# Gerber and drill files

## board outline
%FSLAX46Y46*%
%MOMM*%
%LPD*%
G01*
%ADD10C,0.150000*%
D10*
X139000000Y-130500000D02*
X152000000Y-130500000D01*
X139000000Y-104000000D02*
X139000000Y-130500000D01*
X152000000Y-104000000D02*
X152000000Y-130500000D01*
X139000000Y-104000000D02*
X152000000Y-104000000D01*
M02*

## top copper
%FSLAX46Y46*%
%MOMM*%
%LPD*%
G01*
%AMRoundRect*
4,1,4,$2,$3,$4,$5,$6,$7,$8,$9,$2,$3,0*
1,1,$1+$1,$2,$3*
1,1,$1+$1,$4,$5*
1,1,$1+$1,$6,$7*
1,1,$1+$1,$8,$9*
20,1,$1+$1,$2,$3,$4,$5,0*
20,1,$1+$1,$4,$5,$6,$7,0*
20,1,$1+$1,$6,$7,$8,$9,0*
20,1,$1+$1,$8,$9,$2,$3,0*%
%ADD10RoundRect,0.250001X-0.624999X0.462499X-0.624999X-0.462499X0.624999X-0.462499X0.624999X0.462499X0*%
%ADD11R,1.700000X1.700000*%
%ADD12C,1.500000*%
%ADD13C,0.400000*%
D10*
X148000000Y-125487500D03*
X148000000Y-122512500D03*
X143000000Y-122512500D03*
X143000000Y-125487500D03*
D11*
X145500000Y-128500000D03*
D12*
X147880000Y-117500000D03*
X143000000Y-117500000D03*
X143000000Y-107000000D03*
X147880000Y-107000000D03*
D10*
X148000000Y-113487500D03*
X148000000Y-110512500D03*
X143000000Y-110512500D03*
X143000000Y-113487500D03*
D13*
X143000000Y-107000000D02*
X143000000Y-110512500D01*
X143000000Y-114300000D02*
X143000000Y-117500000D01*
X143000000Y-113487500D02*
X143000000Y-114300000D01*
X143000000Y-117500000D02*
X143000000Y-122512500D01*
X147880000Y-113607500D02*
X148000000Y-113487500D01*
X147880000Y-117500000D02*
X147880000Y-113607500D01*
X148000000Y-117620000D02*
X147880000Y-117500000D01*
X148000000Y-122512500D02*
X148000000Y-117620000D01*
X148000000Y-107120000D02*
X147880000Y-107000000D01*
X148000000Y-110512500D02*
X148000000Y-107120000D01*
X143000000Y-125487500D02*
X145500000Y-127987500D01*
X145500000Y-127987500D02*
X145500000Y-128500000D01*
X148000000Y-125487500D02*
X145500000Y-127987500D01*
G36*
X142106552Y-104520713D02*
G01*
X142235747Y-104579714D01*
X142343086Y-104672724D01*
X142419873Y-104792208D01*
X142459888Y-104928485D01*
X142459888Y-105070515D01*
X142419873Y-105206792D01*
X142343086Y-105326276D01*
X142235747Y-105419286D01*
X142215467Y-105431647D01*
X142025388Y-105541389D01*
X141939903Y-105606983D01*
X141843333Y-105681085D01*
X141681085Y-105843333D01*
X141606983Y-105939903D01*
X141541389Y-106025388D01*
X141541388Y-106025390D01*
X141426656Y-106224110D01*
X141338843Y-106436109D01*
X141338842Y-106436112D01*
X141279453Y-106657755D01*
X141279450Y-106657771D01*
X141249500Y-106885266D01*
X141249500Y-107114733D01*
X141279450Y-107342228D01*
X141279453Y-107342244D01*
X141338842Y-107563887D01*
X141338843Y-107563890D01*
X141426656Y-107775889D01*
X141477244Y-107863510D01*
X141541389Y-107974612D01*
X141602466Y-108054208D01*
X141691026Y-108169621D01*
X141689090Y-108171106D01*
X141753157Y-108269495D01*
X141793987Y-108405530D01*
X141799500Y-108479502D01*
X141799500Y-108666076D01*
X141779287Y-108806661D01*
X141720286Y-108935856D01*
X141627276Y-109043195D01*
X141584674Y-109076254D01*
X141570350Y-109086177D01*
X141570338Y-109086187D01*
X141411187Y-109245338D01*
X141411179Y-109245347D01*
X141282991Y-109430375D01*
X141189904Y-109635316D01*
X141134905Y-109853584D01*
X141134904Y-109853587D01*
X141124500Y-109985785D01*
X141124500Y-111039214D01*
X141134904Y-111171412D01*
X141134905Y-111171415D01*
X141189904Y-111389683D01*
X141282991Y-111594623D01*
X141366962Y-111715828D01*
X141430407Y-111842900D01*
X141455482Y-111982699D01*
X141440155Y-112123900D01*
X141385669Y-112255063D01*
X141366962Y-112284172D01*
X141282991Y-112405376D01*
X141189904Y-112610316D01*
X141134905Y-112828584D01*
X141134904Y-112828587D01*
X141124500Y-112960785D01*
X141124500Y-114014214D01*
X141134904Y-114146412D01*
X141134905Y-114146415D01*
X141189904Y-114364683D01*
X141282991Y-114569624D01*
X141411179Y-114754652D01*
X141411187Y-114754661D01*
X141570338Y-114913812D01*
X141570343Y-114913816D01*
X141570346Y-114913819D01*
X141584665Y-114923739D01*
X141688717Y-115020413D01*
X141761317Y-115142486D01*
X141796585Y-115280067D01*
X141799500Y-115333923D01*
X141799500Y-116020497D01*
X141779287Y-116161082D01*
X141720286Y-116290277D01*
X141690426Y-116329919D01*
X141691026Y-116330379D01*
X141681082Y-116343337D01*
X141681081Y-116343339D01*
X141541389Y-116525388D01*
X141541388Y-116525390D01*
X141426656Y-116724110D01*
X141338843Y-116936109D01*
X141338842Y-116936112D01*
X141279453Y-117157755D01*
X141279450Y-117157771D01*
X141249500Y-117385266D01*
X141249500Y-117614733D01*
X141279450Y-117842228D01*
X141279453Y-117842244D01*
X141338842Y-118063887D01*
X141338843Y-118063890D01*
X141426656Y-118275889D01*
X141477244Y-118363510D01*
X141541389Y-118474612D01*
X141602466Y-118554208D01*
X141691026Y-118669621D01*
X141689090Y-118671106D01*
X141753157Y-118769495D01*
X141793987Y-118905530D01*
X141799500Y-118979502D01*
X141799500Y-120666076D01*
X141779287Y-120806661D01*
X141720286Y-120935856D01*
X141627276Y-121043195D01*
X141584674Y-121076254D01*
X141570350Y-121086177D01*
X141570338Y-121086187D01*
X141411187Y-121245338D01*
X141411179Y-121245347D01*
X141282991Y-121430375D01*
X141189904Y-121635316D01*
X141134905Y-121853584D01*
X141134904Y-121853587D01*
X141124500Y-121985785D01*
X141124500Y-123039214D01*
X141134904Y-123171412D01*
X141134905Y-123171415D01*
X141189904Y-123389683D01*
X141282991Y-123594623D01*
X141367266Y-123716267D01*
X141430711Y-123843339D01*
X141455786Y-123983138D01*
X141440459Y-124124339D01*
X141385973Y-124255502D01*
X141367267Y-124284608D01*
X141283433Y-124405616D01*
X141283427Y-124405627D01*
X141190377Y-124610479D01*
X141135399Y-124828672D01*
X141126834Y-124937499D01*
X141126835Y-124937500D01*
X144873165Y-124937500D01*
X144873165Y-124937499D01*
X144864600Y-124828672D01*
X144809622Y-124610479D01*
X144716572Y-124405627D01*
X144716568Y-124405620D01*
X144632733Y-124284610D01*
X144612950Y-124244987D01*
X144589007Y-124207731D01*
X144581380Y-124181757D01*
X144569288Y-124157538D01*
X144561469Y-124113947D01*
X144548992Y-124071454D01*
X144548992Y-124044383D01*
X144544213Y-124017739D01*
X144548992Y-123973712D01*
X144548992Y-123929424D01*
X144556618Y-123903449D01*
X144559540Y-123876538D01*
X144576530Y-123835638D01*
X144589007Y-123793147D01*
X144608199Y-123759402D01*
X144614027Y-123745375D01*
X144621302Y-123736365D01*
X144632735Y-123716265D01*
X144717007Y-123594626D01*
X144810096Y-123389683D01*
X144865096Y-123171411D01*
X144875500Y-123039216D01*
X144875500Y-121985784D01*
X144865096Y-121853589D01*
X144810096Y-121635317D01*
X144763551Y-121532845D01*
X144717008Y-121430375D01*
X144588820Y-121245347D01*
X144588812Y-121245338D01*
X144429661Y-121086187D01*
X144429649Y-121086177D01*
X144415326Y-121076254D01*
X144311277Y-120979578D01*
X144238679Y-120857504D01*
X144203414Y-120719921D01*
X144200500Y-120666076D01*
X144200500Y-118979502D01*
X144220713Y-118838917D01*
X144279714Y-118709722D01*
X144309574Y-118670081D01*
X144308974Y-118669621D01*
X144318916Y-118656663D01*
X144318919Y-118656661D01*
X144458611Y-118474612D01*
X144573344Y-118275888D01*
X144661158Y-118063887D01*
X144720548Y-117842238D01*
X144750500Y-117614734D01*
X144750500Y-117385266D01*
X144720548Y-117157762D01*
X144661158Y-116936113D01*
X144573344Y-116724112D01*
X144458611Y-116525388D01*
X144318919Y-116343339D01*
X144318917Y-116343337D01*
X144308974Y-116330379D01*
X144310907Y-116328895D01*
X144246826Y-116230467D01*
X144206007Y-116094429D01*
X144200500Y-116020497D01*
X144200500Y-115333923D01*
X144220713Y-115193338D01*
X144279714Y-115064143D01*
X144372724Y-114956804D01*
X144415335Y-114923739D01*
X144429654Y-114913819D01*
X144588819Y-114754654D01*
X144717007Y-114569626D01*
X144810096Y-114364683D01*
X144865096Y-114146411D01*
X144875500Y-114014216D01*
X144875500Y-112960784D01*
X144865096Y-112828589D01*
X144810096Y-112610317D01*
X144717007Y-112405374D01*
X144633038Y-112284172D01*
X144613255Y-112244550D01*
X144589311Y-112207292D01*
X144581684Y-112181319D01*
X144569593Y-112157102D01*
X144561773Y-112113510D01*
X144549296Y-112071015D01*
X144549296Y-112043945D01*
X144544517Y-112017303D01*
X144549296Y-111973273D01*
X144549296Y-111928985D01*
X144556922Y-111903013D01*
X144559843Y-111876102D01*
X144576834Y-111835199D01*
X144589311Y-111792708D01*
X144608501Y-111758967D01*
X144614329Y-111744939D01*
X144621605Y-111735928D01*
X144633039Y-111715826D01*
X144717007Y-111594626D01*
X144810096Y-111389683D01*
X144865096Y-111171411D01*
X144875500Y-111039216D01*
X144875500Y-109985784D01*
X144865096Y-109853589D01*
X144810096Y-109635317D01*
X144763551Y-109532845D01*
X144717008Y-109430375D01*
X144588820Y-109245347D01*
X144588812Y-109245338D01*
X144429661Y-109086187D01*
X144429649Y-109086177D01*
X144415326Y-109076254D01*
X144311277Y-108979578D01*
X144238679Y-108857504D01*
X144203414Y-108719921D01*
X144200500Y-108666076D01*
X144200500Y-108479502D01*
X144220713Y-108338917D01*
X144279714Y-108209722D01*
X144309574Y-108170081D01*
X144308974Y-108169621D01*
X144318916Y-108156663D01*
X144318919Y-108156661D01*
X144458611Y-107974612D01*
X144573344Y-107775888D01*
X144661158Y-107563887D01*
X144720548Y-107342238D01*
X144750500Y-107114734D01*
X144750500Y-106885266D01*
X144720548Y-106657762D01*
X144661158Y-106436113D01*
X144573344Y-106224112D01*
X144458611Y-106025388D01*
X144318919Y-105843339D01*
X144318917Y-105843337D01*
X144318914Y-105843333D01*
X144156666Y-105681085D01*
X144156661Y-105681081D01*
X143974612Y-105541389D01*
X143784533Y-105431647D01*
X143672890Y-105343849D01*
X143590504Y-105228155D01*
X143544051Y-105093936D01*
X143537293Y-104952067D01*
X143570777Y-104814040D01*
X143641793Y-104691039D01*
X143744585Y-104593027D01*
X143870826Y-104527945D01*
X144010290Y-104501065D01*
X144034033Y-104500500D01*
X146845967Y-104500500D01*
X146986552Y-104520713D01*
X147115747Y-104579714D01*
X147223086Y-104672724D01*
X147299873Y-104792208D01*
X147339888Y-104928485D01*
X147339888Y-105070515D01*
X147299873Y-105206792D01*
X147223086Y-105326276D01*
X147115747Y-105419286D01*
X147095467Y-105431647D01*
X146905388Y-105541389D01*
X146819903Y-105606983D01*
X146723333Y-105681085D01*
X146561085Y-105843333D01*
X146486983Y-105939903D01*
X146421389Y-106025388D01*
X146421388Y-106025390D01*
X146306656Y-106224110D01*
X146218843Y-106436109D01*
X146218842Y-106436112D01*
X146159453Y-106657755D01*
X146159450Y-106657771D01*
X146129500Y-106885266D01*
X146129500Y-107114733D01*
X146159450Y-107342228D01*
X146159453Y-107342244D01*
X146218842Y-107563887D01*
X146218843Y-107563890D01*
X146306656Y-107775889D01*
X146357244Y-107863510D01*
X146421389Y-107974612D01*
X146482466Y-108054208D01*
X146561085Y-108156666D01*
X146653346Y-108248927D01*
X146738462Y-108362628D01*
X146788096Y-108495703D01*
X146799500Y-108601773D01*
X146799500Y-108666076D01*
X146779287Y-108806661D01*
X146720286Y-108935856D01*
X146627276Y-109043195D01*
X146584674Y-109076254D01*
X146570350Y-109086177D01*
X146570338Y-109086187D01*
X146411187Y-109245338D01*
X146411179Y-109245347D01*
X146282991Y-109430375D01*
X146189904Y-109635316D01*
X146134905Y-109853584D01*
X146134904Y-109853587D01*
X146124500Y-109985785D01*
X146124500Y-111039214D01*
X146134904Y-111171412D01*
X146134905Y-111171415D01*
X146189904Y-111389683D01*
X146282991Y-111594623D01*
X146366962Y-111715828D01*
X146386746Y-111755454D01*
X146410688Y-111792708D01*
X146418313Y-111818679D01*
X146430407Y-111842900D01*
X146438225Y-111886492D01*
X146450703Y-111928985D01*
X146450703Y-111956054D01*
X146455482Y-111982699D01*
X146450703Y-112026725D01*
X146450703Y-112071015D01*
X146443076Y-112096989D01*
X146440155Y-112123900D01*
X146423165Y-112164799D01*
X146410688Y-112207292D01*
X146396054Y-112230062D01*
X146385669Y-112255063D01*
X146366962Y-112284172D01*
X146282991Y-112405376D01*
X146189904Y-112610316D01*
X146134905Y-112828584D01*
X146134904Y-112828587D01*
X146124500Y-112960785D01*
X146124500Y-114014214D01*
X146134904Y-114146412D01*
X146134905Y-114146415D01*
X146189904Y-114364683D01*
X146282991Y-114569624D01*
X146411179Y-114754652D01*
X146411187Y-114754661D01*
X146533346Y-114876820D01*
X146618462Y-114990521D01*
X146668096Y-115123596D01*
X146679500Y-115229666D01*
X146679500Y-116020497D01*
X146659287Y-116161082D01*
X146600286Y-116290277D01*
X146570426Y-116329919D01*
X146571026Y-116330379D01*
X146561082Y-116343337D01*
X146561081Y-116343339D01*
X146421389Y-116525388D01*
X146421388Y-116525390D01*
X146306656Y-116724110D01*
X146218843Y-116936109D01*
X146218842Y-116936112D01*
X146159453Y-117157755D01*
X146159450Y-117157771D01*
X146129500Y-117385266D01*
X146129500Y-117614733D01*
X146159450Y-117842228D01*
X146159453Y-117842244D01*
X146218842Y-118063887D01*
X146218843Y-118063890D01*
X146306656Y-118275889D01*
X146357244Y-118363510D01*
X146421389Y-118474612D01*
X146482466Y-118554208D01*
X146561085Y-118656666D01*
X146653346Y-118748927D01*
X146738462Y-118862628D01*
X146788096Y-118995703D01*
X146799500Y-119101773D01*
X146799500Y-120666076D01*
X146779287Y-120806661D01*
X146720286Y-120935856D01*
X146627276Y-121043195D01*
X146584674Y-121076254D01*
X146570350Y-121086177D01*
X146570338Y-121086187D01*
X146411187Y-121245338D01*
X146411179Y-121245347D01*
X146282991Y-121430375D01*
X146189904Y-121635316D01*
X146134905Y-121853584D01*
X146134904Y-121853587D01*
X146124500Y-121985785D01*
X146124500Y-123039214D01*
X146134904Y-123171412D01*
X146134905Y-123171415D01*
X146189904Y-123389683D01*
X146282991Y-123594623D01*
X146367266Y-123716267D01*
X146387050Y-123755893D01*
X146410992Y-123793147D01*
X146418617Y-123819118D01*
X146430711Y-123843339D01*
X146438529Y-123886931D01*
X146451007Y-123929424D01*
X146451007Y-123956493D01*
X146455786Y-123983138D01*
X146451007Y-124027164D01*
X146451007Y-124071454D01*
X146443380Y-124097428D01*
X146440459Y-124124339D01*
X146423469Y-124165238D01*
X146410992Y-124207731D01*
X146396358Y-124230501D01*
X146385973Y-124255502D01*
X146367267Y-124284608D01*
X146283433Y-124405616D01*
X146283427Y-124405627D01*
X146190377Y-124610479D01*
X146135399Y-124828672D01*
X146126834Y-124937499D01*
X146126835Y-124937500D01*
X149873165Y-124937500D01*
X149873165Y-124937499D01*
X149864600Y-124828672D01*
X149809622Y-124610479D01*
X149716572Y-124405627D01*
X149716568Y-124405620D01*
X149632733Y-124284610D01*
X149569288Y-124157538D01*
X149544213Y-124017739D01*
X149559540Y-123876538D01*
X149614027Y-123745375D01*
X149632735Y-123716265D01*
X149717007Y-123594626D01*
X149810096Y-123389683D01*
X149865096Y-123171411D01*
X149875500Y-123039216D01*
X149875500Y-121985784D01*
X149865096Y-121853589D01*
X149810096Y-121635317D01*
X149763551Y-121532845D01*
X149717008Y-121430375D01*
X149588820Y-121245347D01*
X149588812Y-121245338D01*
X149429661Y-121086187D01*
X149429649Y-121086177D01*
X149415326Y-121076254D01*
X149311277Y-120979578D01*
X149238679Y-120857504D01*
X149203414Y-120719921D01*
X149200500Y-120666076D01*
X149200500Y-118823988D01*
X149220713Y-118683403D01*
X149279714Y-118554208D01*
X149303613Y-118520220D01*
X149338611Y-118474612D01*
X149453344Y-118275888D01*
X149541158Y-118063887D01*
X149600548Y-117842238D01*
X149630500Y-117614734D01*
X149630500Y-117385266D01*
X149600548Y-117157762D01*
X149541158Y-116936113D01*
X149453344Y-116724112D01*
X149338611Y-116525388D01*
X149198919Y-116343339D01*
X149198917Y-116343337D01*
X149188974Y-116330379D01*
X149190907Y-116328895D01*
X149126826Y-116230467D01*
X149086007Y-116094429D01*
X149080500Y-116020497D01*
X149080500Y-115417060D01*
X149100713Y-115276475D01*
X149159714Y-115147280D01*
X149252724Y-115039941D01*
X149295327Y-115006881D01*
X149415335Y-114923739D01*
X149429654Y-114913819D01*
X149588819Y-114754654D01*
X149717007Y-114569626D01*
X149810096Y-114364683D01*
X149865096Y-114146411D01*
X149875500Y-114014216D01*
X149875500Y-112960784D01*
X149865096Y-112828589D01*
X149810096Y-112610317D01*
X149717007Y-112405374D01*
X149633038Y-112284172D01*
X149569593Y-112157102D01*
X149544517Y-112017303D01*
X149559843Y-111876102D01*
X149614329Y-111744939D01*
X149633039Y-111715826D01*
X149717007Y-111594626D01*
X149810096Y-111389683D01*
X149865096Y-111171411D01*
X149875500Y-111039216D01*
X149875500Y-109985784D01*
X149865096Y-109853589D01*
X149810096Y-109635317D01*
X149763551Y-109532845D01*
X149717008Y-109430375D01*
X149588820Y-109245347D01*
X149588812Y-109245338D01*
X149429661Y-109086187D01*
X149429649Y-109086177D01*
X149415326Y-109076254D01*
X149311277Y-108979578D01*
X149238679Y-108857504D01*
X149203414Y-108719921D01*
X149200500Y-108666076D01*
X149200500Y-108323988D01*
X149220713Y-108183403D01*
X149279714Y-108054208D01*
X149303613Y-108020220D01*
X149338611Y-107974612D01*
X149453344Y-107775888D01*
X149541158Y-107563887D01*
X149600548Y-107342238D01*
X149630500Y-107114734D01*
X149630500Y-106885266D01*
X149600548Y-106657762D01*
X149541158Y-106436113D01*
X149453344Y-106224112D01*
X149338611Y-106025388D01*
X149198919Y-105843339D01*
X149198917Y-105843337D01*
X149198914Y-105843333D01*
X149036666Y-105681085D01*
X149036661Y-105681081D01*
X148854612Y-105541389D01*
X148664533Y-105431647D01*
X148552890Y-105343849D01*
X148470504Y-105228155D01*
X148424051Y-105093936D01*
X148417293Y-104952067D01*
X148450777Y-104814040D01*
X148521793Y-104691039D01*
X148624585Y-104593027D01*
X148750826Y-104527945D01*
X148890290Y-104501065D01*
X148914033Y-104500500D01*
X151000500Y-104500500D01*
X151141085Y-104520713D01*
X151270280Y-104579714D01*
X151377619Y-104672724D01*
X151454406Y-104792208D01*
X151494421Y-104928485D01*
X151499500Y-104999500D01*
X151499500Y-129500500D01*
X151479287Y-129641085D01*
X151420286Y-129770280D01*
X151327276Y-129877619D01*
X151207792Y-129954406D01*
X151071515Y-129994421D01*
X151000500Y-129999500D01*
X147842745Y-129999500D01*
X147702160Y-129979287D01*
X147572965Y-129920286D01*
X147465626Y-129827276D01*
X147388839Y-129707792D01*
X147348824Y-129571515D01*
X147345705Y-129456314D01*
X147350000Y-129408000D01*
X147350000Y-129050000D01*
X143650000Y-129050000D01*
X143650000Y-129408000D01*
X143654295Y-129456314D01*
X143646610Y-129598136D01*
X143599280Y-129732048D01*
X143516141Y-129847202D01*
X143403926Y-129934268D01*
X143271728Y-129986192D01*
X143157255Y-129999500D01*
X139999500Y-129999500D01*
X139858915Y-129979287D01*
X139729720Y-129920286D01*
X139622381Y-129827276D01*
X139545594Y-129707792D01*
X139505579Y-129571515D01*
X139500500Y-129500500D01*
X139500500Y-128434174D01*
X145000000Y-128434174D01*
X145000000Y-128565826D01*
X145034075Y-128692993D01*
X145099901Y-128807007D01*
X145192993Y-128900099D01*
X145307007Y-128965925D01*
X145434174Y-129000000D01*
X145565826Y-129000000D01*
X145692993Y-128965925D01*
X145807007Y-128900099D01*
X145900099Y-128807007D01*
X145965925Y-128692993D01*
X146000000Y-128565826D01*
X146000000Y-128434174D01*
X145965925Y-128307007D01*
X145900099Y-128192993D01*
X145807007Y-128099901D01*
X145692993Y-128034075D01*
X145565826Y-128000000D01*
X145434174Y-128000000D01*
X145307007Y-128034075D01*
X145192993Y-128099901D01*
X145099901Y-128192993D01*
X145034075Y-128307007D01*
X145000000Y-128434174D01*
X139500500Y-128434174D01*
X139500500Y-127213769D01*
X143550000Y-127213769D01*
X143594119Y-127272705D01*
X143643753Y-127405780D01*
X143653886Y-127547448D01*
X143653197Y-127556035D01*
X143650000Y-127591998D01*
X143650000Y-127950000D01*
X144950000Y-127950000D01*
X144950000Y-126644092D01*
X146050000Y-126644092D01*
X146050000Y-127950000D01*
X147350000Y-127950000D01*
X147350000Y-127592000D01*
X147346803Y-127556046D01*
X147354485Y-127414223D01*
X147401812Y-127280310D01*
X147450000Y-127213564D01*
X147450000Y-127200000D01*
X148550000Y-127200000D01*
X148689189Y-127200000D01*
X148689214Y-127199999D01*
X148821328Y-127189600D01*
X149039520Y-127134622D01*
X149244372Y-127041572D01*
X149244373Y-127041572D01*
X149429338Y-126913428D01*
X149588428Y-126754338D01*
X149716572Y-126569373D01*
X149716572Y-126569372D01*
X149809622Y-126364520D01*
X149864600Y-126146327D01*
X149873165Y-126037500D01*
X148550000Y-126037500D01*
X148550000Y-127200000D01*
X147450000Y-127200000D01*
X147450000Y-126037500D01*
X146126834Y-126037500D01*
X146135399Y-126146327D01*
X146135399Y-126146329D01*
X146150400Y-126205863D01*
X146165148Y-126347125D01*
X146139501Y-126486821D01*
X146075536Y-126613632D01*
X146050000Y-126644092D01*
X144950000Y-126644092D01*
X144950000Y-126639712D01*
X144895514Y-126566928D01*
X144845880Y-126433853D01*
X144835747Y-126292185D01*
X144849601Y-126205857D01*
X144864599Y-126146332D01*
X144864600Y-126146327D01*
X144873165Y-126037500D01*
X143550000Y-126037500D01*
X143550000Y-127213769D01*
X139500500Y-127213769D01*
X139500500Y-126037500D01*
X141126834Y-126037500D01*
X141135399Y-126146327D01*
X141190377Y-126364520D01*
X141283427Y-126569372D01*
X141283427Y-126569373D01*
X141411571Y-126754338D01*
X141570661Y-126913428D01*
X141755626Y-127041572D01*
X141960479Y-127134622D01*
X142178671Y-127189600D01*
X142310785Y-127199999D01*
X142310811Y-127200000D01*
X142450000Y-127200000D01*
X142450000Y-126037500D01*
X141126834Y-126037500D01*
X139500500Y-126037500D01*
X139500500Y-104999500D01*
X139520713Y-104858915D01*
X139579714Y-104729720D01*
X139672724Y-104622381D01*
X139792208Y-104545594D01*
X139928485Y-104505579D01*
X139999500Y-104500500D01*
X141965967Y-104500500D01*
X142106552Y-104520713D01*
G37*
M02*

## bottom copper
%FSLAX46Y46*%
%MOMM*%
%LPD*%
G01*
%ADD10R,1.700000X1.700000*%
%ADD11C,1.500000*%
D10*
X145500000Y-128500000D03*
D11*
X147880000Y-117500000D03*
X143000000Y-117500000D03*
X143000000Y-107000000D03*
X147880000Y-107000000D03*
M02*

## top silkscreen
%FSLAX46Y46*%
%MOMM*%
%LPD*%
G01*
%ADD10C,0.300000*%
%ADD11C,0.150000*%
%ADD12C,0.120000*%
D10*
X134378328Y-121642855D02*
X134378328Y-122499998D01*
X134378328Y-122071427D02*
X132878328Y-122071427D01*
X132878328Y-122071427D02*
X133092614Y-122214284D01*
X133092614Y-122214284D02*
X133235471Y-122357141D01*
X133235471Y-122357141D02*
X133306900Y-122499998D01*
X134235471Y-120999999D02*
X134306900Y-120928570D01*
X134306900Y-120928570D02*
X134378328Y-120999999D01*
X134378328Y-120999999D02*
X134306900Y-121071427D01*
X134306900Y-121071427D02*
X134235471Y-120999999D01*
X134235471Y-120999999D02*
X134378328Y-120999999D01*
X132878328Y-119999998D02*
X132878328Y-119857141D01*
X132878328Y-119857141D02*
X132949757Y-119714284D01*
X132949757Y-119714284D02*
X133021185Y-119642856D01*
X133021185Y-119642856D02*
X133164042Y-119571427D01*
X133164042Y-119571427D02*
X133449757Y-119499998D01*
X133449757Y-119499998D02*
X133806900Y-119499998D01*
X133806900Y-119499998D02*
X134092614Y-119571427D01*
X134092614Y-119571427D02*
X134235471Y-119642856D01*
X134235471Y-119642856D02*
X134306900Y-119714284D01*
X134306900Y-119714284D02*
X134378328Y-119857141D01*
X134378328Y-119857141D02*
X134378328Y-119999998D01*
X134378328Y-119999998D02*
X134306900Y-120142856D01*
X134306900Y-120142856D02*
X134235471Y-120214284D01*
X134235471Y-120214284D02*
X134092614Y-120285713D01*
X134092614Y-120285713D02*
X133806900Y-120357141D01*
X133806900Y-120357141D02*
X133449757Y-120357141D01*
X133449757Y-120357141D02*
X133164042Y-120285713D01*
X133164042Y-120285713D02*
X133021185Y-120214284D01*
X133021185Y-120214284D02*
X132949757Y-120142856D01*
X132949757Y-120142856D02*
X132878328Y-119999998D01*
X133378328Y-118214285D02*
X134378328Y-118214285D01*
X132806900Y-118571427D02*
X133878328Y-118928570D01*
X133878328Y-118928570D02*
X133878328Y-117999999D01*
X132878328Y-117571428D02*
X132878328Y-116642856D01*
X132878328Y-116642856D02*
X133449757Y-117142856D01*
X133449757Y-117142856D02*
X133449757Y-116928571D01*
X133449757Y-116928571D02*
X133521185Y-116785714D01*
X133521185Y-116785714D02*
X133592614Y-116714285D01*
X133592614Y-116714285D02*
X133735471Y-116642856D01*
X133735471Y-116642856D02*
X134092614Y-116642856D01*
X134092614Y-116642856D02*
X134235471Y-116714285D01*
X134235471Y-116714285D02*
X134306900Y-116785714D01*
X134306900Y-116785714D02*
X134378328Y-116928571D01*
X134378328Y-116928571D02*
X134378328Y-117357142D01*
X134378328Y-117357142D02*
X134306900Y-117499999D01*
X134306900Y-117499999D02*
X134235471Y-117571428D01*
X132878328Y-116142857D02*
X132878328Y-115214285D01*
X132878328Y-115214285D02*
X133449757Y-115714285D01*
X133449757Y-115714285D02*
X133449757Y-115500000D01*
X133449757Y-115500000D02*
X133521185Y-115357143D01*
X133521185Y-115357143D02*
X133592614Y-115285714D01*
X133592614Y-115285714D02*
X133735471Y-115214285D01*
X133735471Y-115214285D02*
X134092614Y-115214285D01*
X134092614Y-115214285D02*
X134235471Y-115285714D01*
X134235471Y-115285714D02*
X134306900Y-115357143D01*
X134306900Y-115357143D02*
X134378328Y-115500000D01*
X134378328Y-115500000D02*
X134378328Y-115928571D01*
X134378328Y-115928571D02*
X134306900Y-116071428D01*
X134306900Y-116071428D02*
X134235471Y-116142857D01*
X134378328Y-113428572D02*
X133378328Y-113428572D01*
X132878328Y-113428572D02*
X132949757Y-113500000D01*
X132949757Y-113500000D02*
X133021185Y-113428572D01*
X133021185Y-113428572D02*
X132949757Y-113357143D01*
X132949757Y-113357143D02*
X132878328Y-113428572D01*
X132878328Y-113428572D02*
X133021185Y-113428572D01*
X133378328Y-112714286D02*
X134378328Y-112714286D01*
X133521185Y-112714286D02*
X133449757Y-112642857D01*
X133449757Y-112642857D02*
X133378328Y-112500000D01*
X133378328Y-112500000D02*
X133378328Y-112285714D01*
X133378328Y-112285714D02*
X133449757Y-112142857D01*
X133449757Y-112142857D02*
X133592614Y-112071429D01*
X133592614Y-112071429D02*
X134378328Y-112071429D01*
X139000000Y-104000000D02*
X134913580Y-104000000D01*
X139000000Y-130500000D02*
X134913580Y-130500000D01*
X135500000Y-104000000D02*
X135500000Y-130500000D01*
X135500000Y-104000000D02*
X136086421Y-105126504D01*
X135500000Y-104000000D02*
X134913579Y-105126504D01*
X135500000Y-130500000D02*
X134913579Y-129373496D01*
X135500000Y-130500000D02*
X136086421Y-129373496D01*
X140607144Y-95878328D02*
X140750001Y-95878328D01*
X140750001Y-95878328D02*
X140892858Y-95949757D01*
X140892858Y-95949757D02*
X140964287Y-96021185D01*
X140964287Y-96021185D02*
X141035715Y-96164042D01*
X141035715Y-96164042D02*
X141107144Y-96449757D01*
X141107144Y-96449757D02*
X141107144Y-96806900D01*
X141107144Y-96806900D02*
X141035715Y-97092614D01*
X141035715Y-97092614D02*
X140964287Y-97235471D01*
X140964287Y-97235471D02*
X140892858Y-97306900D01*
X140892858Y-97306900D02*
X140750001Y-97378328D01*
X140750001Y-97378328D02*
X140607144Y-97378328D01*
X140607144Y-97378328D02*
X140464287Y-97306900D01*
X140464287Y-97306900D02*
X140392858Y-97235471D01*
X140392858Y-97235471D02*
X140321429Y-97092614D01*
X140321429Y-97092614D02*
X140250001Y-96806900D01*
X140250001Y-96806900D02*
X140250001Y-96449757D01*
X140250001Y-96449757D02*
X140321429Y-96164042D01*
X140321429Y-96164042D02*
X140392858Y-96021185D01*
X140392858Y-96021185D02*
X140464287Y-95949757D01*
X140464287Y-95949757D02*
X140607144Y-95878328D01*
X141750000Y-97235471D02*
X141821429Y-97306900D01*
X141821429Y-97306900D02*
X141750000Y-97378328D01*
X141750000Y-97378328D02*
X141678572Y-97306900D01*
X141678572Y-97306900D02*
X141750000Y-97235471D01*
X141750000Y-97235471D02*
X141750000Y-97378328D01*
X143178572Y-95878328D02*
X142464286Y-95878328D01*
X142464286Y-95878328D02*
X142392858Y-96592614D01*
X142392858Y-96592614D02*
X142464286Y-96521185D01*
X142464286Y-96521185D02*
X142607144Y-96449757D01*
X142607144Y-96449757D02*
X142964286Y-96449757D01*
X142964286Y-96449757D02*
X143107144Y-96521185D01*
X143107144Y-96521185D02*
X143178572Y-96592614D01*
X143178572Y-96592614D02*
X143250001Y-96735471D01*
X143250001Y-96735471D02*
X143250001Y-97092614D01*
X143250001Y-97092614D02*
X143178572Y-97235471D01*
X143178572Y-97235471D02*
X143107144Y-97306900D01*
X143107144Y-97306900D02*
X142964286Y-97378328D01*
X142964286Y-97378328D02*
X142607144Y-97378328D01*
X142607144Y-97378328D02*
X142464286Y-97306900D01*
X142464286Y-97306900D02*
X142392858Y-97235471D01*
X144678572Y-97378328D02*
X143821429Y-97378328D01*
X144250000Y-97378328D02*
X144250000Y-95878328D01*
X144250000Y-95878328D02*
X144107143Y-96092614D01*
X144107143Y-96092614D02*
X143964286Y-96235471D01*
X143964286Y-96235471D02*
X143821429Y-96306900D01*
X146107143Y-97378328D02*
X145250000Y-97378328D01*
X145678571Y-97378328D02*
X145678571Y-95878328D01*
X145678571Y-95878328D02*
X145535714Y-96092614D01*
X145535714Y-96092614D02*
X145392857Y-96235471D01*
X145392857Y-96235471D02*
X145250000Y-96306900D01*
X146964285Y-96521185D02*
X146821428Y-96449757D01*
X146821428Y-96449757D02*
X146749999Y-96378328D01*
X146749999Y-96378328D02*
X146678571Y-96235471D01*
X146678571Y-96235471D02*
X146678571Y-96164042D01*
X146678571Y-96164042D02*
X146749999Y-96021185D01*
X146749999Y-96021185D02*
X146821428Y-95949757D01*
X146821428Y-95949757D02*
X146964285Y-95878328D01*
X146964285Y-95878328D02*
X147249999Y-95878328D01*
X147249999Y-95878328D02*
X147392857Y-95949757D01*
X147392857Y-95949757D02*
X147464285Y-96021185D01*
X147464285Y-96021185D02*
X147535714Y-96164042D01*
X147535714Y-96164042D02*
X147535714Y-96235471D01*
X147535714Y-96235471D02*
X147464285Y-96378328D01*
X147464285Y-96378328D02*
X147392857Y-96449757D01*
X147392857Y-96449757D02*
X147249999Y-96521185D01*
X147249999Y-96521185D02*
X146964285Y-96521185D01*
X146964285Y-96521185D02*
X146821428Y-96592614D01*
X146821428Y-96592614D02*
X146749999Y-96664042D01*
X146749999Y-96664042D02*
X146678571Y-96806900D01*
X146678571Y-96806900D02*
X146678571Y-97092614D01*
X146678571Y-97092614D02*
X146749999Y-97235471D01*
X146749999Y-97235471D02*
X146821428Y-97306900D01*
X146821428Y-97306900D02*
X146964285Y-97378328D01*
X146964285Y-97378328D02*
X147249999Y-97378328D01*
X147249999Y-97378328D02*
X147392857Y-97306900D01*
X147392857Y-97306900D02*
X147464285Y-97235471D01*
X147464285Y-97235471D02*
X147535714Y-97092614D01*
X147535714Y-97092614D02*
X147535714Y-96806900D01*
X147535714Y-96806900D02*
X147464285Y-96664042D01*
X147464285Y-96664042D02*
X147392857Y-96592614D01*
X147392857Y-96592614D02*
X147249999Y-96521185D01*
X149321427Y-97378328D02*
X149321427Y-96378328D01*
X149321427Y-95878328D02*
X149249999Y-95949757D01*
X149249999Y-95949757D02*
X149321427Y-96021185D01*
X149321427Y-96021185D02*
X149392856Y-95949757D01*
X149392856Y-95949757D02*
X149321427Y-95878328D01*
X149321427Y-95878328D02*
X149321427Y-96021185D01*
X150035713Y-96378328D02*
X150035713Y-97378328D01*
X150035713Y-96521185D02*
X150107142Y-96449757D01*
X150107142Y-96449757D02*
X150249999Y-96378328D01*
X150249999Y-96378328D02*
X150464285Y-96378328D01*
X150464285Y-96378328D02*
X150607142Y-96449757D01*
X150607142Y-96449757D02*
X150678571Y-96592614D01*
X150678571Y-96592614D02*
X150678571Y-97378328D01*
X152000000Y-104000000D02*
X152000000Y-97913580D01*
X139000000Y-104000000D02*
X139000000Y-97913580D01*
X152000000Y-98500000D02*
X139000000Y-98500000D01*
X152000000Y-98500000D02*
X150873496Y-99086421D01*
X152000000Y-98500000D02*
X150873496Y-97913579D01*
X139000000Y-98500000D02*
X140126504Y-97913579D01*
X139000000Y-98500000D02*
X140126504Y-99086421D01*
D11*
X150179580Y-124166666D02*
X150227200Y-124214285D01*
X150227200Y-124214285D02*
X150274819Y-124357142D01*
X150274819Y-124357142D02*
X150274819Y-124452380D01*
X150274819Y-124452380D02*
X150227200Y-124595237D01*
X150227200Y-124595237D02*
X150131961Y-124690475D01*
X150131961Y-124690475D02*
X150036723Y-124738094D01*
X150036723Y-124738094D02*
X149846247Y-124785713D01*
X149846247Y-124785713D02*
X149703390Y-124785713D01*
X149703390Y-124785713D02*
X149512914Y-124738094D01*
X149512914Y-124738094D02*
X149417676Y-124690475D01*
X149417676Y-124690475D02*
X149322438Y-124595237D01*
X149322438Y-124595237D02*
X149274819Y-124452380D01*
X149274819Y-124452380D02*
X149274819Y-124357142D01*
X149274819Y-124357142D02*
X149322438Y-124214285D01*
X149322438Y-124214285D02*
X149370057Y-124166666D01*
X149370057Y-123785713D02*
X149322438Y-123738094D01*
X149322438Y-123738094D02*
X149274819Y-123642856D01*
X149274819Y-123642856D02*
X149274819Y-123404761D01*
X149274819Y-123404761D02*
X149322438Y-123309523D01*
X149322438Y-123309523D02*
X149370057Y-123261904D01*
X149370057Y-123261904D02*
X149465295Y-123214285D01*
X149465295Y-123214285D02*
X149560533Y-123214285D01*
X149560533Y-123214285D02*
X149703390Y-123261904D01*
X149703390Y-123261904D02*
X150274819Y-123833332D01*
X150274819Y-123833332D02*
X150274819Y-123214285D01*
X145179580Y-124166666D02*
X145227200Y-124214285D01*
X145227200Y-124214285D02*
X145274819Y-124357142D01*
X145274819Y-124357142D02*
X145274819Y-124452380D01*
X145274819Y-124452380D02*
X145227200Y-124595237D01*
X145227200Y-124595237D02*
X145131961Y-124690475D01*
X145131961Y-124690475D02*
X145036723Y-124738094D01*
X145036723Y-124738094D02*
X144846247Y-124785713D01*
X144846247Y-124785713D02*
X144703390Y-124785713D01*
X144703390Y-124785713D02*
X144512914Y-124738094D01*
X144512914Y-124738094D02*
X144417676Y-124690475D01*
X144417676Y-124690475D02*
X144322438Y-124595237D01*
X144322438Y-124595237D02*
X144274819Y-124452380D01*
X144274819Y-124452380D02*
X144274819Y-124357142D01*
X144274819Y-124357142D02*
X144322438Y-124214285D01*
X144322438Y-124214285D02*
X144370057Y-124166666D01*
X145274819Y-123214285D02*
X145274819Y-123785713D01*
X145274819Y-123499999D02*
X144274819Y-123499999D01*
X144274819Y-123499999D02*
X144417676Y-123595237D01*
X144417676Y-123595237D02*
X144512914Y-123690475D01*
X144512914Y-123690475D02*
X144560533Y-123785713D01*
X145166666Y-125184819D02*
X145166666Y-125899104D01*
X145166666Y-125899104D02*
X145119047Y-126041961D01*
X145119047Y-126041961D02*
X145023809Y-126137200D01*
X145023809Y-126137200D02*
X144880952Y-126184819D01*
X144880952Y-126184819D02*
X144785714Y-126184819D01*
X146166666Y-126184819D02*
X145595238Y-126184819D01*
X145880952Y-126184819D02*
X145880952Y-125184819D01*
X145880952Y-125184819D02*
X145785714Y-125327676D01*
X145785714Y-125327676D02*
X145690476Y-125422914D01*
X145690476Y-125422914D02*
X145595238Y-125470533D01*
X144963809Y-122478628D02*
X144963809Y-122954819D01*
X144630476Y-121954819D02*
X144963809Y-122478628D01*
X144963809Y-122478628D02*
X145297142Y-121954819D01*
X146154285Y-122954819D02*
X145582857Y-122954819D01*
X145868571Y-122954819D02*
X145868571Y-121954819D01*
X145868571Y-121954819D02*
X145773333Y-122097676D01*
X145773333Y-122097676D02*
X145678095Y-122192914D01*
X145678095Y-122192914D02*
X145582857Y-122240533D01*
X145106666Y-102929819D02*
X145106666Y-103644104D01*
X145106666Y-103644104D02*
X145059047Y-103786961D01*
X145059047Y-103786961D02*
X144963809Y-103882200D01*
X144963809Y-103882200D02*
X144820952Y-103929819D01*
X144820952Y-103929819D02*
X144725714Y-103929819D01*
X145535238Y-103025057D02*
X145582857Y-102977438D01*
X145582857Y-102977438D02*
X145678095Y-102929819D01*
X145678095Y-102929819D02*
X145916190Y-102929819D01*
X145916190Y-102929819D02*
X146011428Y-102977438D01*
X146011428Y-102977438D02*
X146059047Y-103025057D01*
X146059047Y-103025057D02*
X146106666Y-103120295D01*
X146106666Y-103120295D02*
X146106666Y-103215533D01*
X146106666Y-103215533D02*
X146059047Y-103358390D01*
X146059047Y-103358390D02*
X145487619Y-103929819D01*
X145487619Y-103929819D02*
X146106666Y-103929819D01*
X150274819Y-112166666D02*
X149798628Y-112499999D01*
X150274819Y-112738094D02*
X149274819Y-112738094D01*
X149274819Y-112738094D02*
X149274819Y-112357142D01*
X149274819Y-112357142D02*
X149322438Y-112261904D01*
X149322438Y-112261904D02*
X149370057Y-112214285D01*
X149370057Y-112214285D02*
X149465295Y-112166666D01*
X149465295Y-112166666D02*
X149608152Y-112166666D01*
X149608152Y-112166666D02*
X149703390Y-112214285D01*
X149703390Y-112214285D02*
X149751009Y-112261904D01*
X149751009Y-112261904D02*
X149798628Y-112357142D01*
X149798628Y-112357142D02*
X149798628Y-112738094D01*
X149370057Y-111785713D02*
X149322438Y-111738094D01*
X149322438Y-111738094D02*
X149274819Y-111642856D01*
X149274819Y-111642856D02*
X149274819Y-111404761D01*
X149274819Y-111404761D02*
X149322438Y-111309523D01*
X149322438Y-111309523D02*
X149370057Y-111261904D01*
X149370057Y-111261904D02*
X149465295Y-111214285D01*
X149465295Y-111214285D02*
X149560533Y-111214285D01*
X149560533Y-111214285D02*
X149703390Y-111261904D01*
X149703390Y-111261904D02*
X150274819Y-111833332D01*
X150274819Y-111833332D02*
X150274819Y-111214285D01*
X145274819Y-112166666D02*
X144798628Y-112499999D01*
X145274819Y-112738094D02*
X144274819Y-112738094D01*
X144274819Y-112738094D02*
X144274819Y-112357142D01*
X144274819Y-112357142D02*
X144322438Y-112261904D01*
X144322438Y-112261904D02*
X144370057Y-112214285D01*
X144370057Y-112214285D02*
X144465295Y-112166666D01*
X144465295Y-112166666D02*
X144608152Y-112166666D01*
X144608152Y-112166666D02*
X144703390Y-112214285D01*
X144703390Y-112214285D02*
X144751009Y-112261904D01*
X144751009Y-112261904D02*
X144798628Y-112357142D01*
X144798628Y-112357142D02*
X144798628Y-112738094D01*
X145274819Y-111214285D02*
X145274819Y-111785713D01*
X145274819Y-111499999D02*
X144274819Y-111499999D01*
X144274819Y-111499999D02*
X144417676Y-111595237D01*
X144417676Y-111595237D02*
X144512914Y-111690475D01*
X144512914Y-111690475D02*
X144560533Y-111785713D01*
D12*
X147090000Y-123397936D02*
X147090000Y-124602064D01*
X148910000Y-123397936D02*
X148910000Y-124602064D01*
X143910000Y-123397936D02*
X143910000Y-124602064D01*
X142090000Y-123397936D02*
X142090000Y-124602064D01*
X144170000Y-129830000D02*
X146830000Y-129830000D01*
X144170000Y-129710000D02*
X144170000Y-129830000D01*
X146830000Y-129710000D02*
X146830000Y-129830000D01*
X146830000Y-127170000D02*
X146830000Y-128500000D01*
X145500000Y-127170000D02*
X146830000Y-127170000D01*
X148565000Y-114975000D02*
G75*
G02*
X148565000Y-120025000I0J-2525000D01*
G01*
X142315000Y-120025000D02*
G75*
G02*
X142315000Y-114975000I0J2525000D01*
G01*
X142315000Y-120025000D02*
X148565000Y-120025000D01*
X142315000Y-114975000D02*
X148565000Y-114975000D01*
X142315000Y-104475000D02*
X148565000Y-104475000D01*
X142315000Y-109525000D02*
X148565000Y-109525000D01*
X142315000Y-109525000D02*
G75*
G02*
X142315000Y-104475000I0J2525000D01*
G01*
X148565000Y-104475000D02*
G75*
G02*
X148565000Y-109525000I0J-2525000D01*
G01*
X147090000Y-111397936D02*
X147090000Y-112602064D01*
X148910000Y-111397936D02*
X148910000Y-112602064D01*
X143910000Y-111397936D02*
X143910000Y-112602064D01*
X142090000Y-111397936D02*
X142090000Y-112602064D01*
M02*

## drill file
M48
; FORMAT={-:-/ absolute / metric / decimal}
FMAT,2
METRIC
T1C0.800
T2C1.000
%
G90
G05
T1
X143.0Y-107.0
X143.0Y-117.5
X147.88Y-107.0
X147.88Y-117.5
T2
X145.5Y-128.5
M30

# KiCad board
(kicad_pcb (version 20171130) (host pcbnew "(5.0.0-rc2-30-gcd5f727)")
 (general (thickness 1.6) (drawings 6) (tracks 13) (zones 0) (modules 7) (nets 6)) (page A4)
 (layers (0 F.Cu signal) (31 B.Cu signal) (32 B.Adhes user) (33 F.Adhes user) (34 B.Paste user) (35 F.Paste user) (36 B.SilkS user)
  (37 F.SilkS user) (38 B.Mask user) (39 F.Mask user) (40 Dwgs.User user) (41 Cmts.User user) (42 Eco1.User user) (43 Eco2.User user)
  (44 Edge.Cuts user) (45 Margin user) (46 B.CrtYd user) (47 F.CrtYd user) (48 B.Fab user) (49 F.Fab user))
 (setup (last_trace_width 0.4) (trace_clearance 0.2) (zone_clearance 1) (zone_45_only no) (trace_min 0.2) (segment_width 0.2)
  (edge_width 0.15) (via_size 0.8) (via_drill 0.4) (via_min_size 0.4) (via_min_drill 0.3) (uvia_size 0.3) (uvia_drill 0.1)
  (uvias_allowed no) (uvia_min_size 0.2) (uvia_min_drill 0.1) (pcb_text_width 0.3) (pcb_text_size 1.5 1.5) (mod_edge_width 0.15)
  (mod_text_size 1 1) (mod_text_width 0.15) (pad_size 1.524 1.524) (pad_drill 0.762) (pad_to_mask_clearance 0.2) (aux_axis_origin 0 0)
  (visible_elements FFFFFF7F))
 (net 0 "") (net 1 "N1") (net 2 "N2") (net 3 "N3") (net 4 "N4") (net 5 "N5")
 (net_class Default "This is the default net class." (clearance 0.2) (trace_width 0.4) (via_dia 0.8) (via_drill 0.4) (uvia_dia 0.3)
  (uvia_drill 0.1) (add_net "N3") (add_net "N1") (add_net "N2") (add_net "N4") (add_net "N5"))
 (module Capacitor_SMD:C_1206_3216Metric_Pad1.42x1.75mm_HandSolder (layer F.Cu) (at 148 124 270)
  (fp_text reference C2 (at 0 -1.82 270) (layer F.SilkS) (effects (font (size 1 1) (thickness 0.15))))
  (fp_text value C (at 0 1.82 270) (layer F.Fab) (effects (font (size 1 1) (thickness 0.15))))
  (fp_line (start -0.602064 0.91) (end 0.602064 0.91) (layer F.SilkS) (width 0.12))
  (fp_line (start -0.602064 -0.91) (end 0.602064 -0.91) (layer F.SilkS) (width 0.12))
  (pad 2 smd roundrect (at 1.4875 0 270) (size 1.425 1.75) (layers F.Cu F.Paste F.Mask) (roundrect_rratio 0.175439) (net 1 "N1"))
  (pad 1 smd roundrect (at -1.4875 0 270) (size 1.425 1.75) (layers F.Cu F.Paste F.Mask) (roundrect_rratio 0.175439) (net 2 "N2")))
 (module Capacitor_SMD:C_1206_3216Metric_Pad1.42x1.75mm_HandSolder (layer F.Cu) (at 143 124 270)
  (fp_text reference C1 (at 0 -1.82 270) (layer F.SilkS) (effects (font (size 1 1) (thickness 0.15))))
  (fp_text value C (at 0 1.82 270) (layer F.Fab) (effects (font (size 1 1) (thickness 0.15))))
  (fp_line (start -0.602064 -0.91) (end 0.602064 -0.91) (layer F.SilkS) (width 0.12))
  (fp_line (start -0.602064 0.91) (end 0.602064 0.91) (layer F.SilkS) (width 0.12))
  (pad 1 smd roundrect (at -1.4875 0 270) (size 1.425 1.75) (layers F.Cu F.Paste F.Mask) (roundrect_rratio 0.175439) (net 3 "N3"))
  (pad 2 smd roundrect (at 1.4875 0 270) (size 1.425 1.75) (layers F.Cu F.Paste F.Mask) (roundrect_rratio 0.175439) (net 1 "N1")))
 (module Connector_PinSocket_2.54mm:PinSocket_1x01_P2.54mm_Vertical (layer F.Cu) (at 145.5 128.5)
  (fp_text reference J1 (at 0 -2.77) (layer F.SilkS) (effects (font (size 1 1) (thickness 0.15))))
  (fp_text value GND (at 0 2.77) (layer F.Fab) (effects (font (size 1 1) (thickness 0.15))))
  (fp_line (start -1.33 1.33) (end 1.33 1.33) (layer F.SilkS) (width 0.12))
  (fp_line (start -1.33 1.21) (end -1.33 1.33) (layer F.SilkS) (width 0.12))
  (fp_line (start 1.33 1.21) (end 1.33 1.33) (layer F.SilkS) (width 0.12))
  (fp_line (start 1.33 -1.33) (end 1.33 0) (layer F.SilkS) (width 0.12))
  (fp_line (start 0 -1.33) (end 1.33 -1.33) (layer F.SilkS) (width 0.12))
  (pad 1 thru_hole rect (at 0 0) (size 1.7 1.7) (drill 1) (layers *.Cu *.Mask) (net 1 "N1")))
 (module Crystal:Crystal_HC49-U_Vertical (layer F.Cu) (at 143 117.5)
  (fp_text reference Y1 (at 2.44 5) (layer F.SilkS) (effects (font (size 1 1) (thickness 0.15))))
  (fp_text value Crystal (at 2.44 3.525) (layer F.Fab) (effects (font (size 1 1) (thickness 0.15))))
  (fp_arc (start 5.565 0) (end 5.565 -2.525) (angle 180) (layer F.SilkS) (width 0.12))
  (fp_arc (start -0.685 0) (end -0.685 -2.525) (angle -180) (layer F.SilkS) (width 0.12))
  (fp_line (start -0.685 2.525) (end 5.565 2.525) (layer F.SilkS) (width 0.12))
  (fp_line (start -0.685 -2.525) (end 5.565 -2.525) (layer F.SilkS) (width 0.12))
  (pad 2 thru_hole circle (at 4.88 0) (size 1.5 1.5) (drill 0.8) (layers *.Cu *.Mask) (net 2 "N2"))
  (pad 1 thru_hole circle (at 0 0) (size 1.5 1.5) (drill 0.8) (layers *.Cu *.Mask) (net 3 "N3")))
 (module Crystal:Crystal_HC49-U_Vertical (layer F.Cu) (at 143 107)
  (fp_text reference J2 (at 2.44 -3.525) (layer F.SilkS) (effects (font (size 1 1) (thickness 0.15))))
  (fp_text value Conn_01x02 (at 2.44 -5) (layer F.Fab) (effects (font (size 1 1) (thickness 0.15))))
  (fp_line (start -0.685 -2.525) (end 5.565 -2.525) (layer F.SilkS) (width 0.12))
  (fp_line (start -0.685 2.525) (end 5.565 2.525) (layer F.SilkS) (width 0.12))
  (fp_arc (start -0.685 0) (end -0.685 -2.525) (angle -180) (layer F.SilkS) (width 0.12))
  (fp_arc (start 5.565 0) (end 5.565 -2.525) (angle 180) (layer F.SilkS) (width 0.12))
  (pad 1 thru_hole circle (at 0 0) (size 1.5 1.5) (drill 0.8) (layers *.Cu *.Mask) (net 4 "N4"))
  (pad 2 thru_hole circle (at 4.88 0) (size 1.5 1.5) (drill 0.8) (layers *.Cu *.Mask) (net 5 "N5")))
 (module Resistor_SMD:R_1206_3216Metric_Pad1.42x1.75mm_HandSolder (layer F.Cu) (at 148 112 270)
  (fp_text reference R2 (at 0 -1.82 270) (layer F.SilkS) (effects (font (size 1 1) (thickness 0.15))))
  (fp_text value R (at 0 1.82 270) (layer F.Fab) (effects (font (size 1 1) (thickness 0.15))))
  (fp_line (start -0.602064 0.91) (end 0.602064 0.91) (layer F.SilkS) (width 0.12))
  (fp_line (start -0.602064 -0.91) (end 0.602064 -0.91) (layer F.SilkS) (width 0.12))
  (pad 2 smd roundrect (at 1.4875 0 270) (size 1.425 1.75) (layers F.Cu F.Paste F.Mask) (roundrect_rratio 0.175439) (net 2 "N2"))
  (pad 1 smd roundrect (at -1.4875 0 270) (size 1.425 1.75) (layers F.Cu F.Paste F.Mask) (roundrect_rratio 0.175439) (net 5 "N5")))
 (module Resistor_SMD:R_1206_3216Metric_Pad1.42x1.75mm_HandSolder (layer F.Cu) (at 143 112 270)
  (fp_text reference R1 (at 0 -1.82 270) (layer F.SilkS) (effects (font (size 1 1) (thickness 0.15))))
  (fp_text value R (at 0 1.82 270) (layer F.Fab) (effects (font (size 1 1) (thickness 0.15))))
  (fp_line (start -0.602064 -0.91) (end 0.602064 -0.91) (layer F.SilkS) (width 0.12))
  (fp_line (start -0.602064 0.91) (end 0.602064 0.91) (layer F.SilkS) (width 0.12))
  (pad 1 smd roundrect (at -1.4875 0 270) (size 1.425 1.75) (layers F.Cu F.Paste F.Mask) (roundrect_rratio 0.175439) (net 4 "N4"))
  (pad 2 smd roundrect (at 1.4875 0 270) (size 1.425 1.75) (layers F.Cu F.Paste F.Mask) (roundrect_rratio 0.175439) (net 3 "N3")))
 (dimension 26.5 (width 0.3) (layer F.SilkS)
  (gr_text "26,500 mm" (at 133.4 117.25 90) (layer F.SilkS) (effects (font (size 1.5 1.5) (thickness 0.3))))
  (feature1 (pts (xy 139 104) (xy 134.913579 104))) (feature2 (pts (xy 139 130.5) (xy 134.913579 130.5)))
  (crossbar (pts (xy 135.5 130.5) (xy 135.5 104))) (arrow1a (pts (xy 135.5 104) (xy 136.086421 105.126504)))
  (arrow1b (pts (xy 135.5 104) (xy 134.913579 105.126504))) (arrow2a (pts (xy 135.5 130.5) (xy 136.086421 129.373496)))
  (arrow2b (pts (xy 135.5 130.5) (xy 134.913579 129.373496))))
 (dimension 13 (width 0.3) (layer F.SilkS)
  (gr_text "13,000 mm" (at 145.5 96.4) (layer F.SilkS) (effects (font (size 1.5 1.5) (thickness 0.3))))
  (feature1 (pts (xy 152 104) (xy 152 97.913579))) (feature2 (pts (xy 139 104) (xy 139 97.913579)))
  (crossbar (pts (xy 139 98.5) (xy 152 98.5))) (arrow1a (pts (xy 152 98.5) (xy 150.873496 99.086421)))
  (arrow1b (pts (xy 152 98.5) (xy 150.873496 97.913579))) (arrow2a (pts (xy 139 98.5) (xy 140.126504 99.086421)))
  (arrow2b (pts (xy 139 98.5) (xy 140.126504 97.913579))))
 (gr_line (start 139 130.5) (end 152 130.5) (layer Edge.Cuts) (width 0.15))
 (gr_line (start 139 104) (end 139 130.5) (layer Edge.Cuts) (width 0.15))
 (gr_line (start 152 104) (end 152 130.5) (layer Edge.Cuts) (width 0.15))
 (gr_line (start 139 104) (end 152 104) (layer Edge.Cuts) (width 0.15))
 (segment (start 143 107) (end 143 110.5125) (width 0.4) (layer F.Cu) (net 4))
 (segment (start 143 114.3) (end 143 117.5) (width 0.4) (layer F.Cu) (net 3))
 (segment (start 143 113.4875) (end 143 114.3) (width 0.4) (layer F.Cu) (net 3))
 (segment (start 143 117.5) (end 143 122.5125) (width 0.4) (layer F.Cu) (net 3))
 (segment (start 147.88 113.6075) (end 148 113.4875) (width 0.4) (layer F.Cu) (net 2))
 (segment (start 147.88 117.5) (end 147.88 113.6075) (width 0.4) (layer F.Cu) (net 2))
 (segment (start 148 117.62) (end 147.88 117.5) (width 0.4) (layer F.Cu) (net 2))
 (segment (start 148 122.5125) (end 148 117.62) (width 0.4) (layer F.Cu) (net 2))
 (segment (start 148 107.12) (end 147.88 107) (width 0.4) (layer F.Cu) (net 5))
 (segment (start 148 110.5125) (end 148 107.12) (width 0.4) (layer F.Cu) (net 5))
 (segment (start 143 125.4875) (end 145.5 127.9875) (width 0.4) (layer F.Cu) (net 1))
 (segment (start 145.5 127.9875) (end 145.5 128.5) (width 0.4) (layer F.Cu) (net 1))
 (segment (start 148 125.4875) (end 145.5 127.9875) (width 0.4) (layer F.Cu) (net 1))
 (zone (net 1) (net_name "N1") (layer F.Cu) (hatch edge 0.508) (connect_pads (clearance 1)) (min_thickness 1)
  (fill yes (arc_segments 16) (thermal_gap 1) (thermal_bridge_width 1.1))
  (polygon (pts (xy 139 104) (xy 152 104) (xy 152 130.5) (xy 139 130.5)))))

